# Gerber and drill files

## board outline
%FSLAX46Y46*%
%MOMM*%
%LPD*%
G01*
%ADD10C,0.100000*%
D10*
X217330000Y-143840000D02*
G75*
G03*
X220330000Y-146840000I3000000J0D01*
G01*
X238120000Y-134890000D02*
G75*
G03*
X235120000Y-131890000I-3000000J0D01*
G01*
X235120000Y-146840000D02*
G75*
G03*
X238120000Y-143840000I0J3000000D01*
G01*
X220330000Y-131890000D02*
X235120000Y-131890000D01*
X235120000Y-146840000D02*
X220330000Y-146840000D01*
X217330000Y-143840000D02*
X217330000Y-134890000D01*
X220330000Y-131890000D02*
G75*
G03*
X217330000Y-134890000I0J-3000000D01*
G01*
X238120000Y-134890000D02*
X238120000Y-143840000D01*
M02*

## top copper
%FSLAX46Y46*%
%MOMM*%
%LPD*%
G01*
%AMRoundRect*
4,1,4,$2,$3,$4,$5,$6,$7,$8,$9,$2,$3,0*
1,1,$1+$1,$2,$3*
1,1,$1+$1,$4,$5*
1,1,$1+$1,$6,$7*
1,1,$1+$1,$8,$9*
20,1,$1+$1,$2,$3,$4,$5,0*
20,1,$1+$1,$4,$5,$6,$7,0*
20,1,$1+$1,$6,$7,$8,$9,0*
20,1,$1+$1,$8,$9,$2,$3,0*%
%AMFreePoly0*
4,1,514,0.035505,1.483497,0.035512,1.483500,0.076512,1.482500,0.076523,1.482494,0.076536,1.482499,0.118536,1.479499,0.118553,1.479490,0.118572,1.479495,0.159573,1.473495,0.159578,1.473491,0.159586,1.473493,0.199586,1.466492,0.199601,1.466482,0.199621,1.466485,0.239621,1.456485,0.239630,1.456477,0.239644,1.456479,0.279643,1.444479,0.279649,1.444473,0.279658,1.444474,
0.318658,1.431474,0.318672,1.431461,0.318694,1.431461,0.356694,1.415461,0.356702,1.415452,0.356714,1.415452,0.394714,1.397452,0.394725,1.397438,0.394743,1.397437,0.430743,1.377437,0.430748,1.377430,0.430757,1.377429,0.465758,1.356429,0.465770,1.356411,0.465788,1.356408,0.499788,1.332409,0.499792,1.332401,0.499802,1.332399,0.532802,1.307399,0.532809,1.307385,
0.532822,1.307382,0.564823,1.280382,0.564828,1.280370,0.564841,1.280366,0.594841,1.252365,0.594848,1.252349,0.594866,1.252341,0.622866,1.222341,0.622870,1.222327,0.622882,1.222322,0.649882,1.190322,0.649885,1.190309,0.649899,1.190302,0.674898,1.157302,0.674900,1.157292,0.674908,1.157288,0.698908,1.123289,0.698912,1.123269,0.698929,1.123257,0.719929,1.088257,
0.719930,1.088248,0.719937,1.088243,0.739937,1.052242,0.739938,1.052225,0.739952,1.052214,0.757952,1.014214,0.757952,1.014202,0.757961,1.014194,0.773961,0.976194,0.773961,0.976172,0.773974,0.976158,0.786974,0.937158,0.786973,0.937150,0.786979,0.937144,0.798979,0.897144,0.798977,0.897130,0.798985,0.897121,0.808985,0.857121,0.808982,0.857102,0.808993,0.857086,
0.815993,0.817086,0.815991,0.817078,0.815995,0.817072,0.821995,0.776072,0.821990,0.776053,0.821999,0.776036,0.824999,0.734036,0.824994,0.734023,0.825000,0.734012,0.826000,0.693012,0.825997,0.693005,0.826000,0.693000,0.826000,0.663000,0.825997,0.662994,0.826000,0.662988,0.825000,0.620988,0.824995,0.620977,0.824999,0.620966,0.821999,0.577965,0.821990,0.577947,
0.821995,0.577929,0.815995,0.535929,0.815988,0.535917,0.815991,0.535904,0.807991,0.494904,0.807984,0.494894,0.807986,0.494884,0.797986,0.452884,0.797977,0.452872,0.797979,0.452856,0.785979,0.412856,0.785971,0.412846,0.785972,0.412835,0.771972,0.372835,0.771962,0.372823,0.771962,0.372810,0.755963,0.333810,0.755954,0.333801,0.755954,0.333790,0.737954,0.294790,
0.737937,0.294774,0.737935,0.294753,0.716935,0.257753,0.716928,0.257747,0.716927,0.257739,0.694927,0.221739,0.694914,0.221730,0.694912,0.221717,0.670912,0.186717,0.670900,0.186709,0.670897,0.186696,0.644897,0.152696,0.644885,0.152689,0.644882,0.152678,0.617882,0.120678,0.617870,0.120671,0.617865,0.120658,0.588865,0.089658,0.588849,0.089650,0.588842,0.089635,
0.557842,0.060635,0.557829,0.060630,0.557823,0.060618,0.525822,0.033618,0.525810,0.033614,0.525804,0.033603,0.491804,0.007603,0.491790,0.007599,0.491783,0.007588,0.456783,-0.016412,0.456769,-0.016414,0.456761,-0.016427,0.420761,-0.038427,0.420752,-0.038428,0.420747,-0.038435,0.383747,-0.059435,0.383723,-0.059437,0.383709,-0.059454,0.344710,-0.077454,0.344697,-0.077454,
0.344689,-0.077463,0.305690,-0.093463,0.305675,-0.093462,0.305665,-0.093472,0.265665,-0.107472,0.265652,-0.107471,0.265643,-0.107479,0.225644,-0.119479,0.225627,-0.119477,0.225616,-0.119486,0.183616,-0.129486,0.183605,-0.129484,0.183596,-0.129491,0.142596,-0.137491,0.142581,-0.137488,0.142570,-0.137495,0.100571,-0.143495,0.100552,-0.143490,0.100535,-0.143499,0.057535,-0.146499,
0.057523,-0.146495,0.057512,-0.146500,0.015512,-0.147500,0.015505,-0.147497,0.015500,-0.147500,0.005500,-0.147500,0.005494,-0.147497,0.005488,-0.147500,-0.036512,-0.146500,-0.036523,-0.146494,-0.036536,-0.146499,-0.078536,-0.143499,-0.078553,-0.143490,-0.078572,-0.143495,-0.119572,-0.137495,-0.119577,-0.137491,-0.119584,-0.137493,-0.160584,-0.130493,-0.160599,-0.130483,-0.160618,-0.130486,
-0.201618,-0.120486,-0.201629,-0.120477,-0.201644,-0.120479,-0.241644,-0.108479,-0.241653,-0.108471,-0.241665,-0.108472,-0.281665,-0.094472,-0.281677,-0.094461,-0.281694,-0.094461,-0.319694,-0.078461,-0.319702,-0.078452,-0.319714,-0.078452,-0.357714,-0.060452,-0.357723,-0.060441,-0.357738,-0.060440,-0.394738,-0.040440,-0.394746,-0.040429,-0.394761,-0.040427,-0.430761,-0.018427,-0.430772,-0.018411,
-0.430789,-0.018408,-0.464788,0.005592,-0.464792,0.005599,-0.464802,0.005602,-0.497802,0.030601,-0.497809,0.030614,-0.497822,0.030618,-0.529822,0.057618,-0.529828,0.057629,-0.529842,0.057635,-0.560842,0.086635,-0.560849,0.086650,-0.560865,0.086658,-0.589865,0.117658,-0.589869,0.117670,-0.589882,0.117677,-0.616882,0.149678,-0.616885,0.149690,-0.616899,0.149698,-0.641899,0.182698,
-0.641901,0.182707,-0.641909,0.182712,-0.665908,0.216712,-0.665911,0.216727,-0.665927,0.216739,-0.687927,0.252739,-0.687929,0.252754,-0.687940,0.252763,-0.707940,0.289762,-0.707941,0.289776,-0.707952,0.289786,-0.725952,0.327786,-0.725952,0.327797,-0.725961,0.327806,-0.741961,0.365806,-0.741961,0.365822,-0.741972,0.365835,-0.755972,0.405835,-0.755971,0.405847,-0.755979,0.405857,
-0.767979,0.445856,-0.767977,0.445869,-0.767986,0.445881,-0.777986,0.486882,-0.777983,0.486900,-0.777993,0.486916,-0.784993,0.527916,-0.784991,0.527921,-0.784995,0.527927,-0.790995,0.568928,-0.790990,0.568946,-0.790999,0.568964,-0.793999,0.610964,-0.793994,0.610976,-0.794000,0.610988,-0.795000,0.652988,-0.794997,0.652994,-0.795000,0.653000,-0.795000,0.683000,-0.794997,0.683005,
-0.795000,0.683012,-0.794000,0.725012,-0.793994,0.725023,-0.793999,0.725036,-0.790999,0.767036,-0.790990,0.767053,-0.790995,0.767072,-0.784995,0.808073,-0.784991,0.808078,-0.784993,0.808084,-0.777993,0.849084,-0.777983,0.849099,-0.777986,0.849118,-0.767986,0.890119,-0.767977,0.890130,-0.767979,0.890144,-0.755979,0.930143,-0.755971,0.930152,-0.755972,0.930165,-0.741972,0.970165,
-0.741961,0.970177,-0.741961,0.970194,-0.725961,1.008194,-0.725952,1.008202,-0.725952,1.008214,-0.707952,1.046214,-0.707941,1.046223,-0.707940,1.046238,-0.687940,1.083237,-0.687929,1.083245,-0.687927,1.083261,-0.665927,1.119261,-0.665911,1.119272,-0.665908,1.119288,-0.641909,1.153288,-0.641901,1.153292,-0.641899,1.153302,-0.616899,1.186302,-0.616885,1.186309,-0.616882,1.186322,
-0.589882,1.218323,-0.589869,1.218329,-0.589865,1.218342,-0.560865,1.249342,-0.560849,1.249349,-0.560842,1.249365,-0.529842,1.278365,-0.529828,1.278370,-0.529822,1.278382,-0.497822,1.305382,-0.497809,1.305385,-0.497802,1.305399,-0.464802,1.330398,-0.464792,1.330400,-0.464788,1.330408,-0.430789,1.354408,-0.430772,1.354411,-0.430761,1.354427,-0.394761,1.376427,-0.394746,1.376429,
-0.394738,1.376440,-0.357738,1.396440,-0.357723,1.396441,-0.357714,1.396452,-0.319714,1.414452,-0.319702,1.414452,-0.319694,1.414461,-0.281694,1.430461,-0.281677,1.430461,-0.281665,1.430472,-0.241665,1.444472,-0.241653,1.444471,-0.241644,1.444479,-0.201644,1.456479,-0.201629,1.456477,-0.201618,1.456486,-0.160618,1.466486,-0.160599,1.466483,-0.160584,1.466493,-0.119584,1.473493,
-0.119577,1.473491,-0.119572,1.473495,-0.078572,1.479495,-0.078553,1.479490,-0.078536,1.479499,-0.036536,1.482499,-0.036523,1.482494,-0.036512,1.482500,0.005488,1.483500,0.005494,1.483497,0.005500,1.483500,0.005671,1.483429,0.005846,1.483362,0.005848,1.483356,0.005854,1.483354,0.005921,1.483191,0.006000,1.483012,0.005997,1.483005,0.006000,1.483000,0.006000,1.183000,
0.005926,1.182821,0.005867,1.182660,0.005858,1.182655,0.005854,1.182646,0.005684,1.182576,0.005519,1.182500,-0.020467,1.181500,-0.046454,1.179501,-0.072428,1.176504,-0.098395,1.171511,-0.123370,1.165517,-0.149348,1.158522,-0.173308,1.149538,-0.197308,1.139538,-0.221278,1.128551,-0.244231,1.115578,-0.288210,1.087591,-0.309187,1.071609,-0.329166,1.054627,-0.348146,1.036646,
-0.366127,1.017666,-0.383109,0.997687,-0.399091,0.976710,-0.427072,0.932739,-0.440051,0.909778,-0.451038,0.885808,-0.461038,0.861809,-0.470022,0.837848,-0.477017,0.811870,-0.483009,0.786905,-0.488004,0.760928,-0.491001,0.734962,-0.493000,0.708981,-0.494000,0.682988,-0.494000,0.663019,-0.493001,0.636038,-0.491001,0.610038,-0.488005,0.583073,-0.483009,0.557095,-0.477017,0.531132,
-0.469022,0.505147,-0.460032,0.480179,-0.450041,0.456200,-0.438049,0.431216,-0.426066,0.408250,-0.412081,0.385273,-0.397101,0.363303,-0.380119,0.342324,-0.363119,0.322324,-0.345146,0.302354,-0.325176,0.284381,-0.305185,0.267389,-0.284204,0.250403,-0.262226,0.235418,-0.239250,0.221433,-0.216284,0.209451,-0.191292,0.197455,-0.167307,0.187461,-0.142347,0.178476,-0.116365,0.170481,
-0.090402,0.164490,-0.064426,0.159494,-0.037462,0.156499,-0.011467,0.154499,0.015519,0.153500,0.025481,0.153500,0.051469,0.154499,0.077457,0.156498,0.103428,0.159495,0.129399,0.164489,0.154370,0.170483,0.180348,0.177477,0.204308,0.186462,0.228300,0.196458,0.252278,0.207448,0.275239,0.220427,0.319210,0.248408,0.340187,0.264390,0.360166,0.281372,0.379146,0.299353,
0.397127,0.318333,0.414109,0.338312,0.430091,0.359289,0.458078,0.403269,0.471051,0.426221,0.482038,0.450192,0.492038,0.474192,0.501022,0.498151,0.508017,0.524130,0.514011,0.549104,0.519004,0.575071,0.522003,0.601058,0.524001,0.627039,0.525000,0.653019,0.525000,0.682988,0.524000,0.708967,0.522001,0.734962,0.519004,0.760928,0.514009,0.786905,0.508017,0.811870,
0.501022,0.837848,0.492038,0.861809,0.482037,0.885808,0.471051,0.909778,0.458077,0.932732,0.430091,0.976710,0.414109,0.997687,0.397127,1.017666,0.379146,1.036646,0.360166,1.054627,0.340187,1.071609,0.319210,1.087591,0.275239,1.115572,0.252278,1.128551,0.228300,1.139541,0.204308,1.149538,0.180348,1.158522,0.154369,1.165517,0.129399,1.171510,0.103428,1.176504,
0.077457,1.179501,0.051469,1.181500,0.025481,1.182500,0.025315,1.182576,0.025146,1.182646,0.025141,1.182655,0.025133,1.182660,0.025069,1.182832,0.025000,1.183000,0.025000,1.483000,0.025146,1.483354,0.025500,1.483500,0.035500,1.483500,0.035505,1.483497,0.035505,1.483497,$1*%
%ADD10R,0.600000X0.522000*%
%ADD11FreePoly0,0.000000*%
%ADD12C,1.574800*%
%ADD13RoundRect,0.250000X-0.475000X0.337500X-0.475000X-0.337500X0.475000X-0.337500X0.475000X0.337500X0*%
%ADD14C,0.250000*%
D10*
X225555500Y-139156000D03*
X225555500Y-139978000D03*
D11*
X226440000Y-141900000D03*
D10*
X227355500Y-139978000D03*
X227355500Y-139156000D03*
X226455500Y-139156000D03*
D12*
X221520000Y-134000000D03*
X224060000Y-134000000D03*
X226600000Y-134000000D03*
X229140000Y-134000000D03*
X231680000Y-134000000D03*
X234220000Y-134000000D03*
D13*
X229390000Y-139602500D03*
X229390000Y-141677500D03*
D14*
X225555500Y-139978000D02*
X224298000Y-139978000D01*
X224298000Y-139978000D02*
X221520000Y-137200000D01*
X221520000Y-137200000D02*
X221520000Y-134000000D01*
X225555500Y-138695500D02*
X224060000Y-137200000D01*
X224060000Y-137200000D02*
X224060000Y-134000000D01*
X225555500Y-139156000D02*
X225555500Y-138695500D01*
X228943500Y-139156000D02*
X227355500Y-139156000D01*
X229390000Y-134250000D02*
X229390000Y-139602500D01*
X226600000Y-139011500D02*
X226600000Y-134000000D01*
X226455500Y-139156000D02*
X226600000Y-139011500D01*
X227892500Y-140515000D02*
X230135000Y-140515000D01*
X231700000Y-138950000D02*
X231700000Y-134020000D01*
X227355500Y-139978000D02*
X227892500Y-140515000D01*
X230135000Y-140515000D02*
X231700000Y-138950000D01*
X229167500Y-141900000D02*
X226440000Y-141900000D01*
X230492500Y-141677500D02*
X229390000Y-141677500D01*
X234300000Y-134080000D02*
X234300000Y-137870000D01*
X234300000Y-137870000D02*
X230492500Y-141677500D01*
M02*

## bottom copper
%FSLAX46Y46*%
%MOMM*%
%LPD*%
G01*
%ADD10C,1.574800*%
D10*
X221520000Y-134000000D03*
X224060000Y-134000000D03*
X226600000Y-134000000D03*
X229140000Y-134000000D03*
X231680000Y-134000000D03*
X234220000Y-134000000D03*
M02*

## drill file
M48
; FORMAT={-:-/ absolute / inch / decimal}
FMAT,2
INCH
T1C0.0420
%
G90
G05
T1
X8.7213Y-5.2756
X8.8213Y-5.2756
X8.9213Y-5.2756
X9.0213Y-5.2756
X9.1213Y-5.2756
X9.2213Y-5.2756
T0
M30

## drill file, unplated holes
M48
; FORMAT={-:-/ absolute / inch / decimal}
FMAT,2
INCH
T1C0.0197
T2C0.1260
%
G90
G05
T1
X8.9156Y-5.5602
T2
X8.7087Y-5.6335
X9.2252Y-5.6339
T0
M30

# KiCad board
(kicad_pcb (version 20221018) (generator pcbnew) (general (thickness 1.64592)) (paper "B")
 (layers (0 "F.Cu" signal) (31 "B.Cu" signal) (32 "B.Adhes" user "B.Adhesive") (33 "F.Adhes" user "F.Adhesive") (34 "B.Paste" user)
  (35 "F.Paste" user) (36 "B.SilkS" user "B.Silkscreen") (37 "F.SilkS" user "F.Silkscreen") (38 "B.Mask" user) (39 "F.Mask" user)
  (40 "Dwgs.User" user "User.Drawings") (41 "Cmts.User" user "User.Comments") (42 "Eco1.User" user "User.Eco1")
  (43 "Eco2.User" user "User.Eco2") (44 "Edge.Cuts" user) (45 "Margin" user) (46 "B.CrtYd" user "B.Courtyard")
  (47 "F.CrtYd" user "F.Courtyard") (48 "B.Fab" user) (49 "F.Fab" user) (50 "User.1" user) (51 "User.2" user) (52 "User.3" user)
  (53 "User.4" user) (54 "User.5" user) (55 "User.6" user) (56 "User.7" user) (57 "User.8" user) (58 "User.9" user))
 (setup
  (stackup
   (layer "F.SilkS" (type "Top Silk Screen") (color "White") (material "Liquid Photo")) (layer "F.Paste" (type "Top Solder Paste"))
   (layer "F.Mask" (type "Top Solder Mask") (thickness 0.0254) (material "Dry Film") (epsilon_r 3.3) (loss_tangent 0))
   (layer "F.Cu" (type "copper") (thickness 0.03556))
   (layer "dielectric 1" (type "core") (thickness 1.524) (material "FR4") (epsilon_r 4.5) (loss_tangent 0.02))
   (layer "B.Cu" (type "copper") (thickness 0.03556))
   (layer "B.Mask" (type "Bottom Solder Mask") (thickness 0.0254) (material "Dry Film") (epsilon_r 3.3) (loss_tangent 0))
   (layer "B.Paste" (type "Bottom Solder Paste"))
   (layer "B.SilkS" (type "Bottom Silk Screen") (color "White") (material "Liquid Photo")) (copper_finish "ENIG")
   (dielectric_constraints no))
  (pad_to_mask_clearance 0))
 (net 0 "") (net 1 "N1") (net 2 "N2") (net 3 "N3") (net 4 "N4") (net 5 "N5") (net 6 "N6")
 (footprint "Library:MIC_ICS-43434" (layer "F.Cu") (at 226.4555 140.517)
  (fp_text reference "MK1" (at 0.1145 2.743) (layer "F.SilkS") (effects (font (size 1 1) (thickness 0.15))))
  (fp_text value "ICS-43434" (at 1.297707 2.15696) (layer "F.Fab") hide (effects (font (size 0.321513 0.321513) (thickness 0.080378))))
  (pad "" np_thru_hole circle (at 0 0.713) (size 0.5 0.5) (drill 0.5) (layers "*.Cu" "*.Mask"))
  (pad "1" smd rect (at -0.9 -1.361) (size 0.6 0.522) (layers "F.Cu" "F.Mask") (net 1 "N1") (solder_mask_margin 0.102))
  (pad "2" smd rect (at -0.9 -0.539) (size 0.6 0.522) (layers "F.Cu" "F.Mask") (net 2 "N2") (solder_mask_margin 0.102))
  (pad "3" smd custom (at -0.0155 1.383) (size 0.1 0.1) (layers "F.Cu") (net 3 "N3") (thermal_bridge_angle 45)
   (options (clearance outline) (anchor rect)) (primitives))
  (pad "4" smd rect (at 0.9 -0.539) (size 0.6 0.522) (layers "F.Cu" "F.Mask") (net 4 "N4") (solder_mask_margin 0.102))
  (pad "5" smd rect (at 0.9 -1.361) (size 0.6 0.522) (layers "F.Cu" "F.Mask") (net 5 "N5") (solder_mask_margin 0.102))
  (pad "6" smd rect (at 0 -1.361) (size 0.6 0.522) (layers "F.Cu" "F.Mask") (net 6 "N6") (solder_mask_margin 0.102)))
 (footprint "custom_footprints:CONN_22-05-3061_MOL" (layer "F.Cu") (at 221.52 134)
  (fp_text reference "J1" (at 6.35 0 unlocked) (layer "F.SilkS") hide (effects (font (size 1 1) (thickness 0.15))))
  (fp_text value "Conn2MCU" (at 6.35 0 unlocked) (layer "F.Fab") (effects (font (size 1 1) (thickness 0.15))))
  (pad "1" thru_hole circle (at 0 0) (size 1.5748 1.5748) (drill 1.0668) (layers "*.Cu" "*.Mask") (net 2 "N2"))
  (pad "2" thru_hole circle (at 2.54 0) (size 1.5748 1.5748) (drill 1.0668) (layers "*.Cu" "*.Mask") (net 1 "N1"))
  (pad "3" thru_hole circle (at 5.08 0) (size 1.5748 1.5748) (drill 1.0668) (layers "*.Cu" "*.Mask") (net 6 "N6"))
  (pad "4" thru_hole circle (at 7.62 0) (size 1.5748 1.5748) (drill 1.0668) (layers "*.Cu" "*.Mask") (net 5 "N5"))
  (pad "5" thru_hole circle (at 10.16 0) (size 1.5748 1.5748) (drill 1.0668) (layers "*.Cu" "*.Mask") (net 4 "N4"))
  (pad "6" thru_hole circle (at 12.7 0) (size 1.5748 1.5748) (drill 1.0668) (layers "*.Cu" "*.Mask") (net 3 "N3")))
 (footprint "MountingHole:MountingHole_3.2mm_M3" (layer "F.Cu") (at 234.32 143.1)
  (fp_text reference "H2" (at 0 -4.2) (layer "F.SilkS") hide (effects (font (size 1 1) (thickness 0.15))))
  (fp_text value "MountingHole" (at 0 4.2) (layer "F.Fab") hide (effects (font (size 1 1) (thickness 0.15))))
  (pad "" np_thru_hole circle (at 0 0) (size 3.2 3.2) (drill 3.2) (layers "*.Cu" "*.Mask")))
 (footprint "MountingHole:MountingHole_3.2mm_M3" (layer "F.Cu") (at 221.2 143.09)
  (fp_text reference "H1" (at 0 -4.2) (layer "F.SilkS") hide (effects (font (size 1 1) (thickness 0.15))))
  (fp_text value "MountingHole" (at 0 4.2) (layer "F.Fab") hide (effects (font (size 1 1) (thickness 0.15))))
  (pad "" np_thru_hole circle (at 0 0) (size 3.2 3.2) (drill 3.2) (layers "*.Cu" "*.Mask")))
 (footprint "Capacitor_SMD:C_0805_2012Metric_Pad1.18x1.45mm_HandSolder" (layer "F.Cu") (at 229.39 140.64 -90)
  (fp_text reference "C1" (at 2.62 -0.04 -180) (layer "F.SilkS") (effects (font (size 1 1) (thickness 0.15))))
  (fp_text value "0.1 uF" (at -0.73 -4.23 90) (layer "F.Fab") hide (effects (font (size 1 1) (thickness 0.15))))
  (pad "1" smd roundrect (at -1.0375 0 270) (size 1.175 1.45) (layers "F.Cu" "F.Paste" "F.Mask") (roundrect_rratio 0.2127659574)
   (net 5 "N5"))
  (pad "2" smd roundrect (at 1.0375 0 270) (size 1.175 1.45) (layers "F.Cu" "F.Paste" "F.Mask") (roundrect_rratio 0.2127659574) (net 3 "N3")))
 (gr_arc (start 220.33 146.84) (mid 218.20868 145.96132) (end 217.33 143.84) (stroke (width 0.1) (type default)) (layer "Edge.Cuts"))
 (gr_arc (start 235.12 131.89) (mid 237.24132 132.76868) (end 238.12 134.89) (stroke (width 0.1) (type default)) (layer "Edge.Cuts"))
 (gr_arc (start 238.12 143.84) (mid 237.24132 145.96132) (end 235.12 146.84) (stroke (width 0.1) (type default)) (layer "Edge.Cuts"))
 (gr_line (start 220.33 131.89) (end 235.12 131.89) (stroke (width 0.1) (type default)) (layer "Edge.Cuts"))
 (gr_line (start 235.12 146.84) (end 220.33 146.84) (stroke (width 0.1) (type default)) (layer "Edge.Cuts"))
 (gr_line (start 217.33 143.84) (end 217.33 134.89) (stroke (width 0.1) (type default)) (layer "Edge.Cuts"))
 (gr_arc (start 217.33 134.89) (mid 218.20868 132.76868) (end 220.33 131.89) (stroke (width 0.1) (type default)) (layer "Edge.Cuts"))
 (gr_line (start 238.12 134.89) (end 238.12 143.84) (stroke (width 0.1) (type default)) (layer "Edge.Cuts"))
 (segment (start 225.5555 139.978) (end 224.298 139.978) (width 0.25) (layer "F.Cu") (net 2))
 (segment (start 224.298 139.978) (end 221.52 137.2) (width 0.25) (layer "F.Cu") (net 2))
 (segment (start 221.52 137.2) (end 221.52 134) (width 0.25) (layer "F.Cu") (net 2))
 (segment (start 225.5555 138.6955) (end 224.06 137.2) (width 0.25) (layer "F.Cu") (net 1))
 (segment (start 224.06 137.2) (end 224.06 134) (width 0.25) (layer "F.Cu") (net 1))
 (segment (start 225.5555 139.156) (end 225.5555 138.6955) (width 0.25) (layer "F.Cu") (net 1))
 (segment (start 228.9435 139.156) (end 227.3555 139.156) (width 0.25) (layer "F.Cu") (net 5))
 (segment (start 229.39 134.25) (end 229.39 139.6025) (width 0.25) (layer "F.Cu") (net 5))
 (segment (start 226.6 139.0115) (end 226.6 134) (width 0.25) (layer "F.Cu") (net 6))
 (segment (start 226.4555 139.156) (end 226.6 139.0115) (width 0.25) (layer "F.Cu") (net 6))
 (segment (start 227.8925 140.515) (end 230.135 140.515) (width 0.25) (layer "F.Cu") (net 4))
 (segment (start 231.7 138.95) (end 231.7 134.02) (width 0.25) (layer "F.Cu") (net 4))
 (segment (start 227.3555 139.978) (end 227.8925 140.515) (width 0.25) (layer "F.Cu") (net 4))
 (segment (start 230.135 140.515) (end 231.7 138.95) (width 0.25) (layer "F.Cu") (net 4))
 (segment (start 229.1675 141.9) (end 226.44 141.9) (width 0.25) (layer "F.Cu") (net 3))
 (segment (start 230.4925 141.6775) (end 229.39 141.6775) (width 0.25) (layer "F.Cu") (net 3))
 (segment (start 234.3 134.08) (end 234.3 137.87) (width 0.25) (layer "F.Cu") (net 3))
 (segment (start 234.3 137.87) (end 230.4925 141.6775) (width 0.25) (layer "F.Cu") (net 3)))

